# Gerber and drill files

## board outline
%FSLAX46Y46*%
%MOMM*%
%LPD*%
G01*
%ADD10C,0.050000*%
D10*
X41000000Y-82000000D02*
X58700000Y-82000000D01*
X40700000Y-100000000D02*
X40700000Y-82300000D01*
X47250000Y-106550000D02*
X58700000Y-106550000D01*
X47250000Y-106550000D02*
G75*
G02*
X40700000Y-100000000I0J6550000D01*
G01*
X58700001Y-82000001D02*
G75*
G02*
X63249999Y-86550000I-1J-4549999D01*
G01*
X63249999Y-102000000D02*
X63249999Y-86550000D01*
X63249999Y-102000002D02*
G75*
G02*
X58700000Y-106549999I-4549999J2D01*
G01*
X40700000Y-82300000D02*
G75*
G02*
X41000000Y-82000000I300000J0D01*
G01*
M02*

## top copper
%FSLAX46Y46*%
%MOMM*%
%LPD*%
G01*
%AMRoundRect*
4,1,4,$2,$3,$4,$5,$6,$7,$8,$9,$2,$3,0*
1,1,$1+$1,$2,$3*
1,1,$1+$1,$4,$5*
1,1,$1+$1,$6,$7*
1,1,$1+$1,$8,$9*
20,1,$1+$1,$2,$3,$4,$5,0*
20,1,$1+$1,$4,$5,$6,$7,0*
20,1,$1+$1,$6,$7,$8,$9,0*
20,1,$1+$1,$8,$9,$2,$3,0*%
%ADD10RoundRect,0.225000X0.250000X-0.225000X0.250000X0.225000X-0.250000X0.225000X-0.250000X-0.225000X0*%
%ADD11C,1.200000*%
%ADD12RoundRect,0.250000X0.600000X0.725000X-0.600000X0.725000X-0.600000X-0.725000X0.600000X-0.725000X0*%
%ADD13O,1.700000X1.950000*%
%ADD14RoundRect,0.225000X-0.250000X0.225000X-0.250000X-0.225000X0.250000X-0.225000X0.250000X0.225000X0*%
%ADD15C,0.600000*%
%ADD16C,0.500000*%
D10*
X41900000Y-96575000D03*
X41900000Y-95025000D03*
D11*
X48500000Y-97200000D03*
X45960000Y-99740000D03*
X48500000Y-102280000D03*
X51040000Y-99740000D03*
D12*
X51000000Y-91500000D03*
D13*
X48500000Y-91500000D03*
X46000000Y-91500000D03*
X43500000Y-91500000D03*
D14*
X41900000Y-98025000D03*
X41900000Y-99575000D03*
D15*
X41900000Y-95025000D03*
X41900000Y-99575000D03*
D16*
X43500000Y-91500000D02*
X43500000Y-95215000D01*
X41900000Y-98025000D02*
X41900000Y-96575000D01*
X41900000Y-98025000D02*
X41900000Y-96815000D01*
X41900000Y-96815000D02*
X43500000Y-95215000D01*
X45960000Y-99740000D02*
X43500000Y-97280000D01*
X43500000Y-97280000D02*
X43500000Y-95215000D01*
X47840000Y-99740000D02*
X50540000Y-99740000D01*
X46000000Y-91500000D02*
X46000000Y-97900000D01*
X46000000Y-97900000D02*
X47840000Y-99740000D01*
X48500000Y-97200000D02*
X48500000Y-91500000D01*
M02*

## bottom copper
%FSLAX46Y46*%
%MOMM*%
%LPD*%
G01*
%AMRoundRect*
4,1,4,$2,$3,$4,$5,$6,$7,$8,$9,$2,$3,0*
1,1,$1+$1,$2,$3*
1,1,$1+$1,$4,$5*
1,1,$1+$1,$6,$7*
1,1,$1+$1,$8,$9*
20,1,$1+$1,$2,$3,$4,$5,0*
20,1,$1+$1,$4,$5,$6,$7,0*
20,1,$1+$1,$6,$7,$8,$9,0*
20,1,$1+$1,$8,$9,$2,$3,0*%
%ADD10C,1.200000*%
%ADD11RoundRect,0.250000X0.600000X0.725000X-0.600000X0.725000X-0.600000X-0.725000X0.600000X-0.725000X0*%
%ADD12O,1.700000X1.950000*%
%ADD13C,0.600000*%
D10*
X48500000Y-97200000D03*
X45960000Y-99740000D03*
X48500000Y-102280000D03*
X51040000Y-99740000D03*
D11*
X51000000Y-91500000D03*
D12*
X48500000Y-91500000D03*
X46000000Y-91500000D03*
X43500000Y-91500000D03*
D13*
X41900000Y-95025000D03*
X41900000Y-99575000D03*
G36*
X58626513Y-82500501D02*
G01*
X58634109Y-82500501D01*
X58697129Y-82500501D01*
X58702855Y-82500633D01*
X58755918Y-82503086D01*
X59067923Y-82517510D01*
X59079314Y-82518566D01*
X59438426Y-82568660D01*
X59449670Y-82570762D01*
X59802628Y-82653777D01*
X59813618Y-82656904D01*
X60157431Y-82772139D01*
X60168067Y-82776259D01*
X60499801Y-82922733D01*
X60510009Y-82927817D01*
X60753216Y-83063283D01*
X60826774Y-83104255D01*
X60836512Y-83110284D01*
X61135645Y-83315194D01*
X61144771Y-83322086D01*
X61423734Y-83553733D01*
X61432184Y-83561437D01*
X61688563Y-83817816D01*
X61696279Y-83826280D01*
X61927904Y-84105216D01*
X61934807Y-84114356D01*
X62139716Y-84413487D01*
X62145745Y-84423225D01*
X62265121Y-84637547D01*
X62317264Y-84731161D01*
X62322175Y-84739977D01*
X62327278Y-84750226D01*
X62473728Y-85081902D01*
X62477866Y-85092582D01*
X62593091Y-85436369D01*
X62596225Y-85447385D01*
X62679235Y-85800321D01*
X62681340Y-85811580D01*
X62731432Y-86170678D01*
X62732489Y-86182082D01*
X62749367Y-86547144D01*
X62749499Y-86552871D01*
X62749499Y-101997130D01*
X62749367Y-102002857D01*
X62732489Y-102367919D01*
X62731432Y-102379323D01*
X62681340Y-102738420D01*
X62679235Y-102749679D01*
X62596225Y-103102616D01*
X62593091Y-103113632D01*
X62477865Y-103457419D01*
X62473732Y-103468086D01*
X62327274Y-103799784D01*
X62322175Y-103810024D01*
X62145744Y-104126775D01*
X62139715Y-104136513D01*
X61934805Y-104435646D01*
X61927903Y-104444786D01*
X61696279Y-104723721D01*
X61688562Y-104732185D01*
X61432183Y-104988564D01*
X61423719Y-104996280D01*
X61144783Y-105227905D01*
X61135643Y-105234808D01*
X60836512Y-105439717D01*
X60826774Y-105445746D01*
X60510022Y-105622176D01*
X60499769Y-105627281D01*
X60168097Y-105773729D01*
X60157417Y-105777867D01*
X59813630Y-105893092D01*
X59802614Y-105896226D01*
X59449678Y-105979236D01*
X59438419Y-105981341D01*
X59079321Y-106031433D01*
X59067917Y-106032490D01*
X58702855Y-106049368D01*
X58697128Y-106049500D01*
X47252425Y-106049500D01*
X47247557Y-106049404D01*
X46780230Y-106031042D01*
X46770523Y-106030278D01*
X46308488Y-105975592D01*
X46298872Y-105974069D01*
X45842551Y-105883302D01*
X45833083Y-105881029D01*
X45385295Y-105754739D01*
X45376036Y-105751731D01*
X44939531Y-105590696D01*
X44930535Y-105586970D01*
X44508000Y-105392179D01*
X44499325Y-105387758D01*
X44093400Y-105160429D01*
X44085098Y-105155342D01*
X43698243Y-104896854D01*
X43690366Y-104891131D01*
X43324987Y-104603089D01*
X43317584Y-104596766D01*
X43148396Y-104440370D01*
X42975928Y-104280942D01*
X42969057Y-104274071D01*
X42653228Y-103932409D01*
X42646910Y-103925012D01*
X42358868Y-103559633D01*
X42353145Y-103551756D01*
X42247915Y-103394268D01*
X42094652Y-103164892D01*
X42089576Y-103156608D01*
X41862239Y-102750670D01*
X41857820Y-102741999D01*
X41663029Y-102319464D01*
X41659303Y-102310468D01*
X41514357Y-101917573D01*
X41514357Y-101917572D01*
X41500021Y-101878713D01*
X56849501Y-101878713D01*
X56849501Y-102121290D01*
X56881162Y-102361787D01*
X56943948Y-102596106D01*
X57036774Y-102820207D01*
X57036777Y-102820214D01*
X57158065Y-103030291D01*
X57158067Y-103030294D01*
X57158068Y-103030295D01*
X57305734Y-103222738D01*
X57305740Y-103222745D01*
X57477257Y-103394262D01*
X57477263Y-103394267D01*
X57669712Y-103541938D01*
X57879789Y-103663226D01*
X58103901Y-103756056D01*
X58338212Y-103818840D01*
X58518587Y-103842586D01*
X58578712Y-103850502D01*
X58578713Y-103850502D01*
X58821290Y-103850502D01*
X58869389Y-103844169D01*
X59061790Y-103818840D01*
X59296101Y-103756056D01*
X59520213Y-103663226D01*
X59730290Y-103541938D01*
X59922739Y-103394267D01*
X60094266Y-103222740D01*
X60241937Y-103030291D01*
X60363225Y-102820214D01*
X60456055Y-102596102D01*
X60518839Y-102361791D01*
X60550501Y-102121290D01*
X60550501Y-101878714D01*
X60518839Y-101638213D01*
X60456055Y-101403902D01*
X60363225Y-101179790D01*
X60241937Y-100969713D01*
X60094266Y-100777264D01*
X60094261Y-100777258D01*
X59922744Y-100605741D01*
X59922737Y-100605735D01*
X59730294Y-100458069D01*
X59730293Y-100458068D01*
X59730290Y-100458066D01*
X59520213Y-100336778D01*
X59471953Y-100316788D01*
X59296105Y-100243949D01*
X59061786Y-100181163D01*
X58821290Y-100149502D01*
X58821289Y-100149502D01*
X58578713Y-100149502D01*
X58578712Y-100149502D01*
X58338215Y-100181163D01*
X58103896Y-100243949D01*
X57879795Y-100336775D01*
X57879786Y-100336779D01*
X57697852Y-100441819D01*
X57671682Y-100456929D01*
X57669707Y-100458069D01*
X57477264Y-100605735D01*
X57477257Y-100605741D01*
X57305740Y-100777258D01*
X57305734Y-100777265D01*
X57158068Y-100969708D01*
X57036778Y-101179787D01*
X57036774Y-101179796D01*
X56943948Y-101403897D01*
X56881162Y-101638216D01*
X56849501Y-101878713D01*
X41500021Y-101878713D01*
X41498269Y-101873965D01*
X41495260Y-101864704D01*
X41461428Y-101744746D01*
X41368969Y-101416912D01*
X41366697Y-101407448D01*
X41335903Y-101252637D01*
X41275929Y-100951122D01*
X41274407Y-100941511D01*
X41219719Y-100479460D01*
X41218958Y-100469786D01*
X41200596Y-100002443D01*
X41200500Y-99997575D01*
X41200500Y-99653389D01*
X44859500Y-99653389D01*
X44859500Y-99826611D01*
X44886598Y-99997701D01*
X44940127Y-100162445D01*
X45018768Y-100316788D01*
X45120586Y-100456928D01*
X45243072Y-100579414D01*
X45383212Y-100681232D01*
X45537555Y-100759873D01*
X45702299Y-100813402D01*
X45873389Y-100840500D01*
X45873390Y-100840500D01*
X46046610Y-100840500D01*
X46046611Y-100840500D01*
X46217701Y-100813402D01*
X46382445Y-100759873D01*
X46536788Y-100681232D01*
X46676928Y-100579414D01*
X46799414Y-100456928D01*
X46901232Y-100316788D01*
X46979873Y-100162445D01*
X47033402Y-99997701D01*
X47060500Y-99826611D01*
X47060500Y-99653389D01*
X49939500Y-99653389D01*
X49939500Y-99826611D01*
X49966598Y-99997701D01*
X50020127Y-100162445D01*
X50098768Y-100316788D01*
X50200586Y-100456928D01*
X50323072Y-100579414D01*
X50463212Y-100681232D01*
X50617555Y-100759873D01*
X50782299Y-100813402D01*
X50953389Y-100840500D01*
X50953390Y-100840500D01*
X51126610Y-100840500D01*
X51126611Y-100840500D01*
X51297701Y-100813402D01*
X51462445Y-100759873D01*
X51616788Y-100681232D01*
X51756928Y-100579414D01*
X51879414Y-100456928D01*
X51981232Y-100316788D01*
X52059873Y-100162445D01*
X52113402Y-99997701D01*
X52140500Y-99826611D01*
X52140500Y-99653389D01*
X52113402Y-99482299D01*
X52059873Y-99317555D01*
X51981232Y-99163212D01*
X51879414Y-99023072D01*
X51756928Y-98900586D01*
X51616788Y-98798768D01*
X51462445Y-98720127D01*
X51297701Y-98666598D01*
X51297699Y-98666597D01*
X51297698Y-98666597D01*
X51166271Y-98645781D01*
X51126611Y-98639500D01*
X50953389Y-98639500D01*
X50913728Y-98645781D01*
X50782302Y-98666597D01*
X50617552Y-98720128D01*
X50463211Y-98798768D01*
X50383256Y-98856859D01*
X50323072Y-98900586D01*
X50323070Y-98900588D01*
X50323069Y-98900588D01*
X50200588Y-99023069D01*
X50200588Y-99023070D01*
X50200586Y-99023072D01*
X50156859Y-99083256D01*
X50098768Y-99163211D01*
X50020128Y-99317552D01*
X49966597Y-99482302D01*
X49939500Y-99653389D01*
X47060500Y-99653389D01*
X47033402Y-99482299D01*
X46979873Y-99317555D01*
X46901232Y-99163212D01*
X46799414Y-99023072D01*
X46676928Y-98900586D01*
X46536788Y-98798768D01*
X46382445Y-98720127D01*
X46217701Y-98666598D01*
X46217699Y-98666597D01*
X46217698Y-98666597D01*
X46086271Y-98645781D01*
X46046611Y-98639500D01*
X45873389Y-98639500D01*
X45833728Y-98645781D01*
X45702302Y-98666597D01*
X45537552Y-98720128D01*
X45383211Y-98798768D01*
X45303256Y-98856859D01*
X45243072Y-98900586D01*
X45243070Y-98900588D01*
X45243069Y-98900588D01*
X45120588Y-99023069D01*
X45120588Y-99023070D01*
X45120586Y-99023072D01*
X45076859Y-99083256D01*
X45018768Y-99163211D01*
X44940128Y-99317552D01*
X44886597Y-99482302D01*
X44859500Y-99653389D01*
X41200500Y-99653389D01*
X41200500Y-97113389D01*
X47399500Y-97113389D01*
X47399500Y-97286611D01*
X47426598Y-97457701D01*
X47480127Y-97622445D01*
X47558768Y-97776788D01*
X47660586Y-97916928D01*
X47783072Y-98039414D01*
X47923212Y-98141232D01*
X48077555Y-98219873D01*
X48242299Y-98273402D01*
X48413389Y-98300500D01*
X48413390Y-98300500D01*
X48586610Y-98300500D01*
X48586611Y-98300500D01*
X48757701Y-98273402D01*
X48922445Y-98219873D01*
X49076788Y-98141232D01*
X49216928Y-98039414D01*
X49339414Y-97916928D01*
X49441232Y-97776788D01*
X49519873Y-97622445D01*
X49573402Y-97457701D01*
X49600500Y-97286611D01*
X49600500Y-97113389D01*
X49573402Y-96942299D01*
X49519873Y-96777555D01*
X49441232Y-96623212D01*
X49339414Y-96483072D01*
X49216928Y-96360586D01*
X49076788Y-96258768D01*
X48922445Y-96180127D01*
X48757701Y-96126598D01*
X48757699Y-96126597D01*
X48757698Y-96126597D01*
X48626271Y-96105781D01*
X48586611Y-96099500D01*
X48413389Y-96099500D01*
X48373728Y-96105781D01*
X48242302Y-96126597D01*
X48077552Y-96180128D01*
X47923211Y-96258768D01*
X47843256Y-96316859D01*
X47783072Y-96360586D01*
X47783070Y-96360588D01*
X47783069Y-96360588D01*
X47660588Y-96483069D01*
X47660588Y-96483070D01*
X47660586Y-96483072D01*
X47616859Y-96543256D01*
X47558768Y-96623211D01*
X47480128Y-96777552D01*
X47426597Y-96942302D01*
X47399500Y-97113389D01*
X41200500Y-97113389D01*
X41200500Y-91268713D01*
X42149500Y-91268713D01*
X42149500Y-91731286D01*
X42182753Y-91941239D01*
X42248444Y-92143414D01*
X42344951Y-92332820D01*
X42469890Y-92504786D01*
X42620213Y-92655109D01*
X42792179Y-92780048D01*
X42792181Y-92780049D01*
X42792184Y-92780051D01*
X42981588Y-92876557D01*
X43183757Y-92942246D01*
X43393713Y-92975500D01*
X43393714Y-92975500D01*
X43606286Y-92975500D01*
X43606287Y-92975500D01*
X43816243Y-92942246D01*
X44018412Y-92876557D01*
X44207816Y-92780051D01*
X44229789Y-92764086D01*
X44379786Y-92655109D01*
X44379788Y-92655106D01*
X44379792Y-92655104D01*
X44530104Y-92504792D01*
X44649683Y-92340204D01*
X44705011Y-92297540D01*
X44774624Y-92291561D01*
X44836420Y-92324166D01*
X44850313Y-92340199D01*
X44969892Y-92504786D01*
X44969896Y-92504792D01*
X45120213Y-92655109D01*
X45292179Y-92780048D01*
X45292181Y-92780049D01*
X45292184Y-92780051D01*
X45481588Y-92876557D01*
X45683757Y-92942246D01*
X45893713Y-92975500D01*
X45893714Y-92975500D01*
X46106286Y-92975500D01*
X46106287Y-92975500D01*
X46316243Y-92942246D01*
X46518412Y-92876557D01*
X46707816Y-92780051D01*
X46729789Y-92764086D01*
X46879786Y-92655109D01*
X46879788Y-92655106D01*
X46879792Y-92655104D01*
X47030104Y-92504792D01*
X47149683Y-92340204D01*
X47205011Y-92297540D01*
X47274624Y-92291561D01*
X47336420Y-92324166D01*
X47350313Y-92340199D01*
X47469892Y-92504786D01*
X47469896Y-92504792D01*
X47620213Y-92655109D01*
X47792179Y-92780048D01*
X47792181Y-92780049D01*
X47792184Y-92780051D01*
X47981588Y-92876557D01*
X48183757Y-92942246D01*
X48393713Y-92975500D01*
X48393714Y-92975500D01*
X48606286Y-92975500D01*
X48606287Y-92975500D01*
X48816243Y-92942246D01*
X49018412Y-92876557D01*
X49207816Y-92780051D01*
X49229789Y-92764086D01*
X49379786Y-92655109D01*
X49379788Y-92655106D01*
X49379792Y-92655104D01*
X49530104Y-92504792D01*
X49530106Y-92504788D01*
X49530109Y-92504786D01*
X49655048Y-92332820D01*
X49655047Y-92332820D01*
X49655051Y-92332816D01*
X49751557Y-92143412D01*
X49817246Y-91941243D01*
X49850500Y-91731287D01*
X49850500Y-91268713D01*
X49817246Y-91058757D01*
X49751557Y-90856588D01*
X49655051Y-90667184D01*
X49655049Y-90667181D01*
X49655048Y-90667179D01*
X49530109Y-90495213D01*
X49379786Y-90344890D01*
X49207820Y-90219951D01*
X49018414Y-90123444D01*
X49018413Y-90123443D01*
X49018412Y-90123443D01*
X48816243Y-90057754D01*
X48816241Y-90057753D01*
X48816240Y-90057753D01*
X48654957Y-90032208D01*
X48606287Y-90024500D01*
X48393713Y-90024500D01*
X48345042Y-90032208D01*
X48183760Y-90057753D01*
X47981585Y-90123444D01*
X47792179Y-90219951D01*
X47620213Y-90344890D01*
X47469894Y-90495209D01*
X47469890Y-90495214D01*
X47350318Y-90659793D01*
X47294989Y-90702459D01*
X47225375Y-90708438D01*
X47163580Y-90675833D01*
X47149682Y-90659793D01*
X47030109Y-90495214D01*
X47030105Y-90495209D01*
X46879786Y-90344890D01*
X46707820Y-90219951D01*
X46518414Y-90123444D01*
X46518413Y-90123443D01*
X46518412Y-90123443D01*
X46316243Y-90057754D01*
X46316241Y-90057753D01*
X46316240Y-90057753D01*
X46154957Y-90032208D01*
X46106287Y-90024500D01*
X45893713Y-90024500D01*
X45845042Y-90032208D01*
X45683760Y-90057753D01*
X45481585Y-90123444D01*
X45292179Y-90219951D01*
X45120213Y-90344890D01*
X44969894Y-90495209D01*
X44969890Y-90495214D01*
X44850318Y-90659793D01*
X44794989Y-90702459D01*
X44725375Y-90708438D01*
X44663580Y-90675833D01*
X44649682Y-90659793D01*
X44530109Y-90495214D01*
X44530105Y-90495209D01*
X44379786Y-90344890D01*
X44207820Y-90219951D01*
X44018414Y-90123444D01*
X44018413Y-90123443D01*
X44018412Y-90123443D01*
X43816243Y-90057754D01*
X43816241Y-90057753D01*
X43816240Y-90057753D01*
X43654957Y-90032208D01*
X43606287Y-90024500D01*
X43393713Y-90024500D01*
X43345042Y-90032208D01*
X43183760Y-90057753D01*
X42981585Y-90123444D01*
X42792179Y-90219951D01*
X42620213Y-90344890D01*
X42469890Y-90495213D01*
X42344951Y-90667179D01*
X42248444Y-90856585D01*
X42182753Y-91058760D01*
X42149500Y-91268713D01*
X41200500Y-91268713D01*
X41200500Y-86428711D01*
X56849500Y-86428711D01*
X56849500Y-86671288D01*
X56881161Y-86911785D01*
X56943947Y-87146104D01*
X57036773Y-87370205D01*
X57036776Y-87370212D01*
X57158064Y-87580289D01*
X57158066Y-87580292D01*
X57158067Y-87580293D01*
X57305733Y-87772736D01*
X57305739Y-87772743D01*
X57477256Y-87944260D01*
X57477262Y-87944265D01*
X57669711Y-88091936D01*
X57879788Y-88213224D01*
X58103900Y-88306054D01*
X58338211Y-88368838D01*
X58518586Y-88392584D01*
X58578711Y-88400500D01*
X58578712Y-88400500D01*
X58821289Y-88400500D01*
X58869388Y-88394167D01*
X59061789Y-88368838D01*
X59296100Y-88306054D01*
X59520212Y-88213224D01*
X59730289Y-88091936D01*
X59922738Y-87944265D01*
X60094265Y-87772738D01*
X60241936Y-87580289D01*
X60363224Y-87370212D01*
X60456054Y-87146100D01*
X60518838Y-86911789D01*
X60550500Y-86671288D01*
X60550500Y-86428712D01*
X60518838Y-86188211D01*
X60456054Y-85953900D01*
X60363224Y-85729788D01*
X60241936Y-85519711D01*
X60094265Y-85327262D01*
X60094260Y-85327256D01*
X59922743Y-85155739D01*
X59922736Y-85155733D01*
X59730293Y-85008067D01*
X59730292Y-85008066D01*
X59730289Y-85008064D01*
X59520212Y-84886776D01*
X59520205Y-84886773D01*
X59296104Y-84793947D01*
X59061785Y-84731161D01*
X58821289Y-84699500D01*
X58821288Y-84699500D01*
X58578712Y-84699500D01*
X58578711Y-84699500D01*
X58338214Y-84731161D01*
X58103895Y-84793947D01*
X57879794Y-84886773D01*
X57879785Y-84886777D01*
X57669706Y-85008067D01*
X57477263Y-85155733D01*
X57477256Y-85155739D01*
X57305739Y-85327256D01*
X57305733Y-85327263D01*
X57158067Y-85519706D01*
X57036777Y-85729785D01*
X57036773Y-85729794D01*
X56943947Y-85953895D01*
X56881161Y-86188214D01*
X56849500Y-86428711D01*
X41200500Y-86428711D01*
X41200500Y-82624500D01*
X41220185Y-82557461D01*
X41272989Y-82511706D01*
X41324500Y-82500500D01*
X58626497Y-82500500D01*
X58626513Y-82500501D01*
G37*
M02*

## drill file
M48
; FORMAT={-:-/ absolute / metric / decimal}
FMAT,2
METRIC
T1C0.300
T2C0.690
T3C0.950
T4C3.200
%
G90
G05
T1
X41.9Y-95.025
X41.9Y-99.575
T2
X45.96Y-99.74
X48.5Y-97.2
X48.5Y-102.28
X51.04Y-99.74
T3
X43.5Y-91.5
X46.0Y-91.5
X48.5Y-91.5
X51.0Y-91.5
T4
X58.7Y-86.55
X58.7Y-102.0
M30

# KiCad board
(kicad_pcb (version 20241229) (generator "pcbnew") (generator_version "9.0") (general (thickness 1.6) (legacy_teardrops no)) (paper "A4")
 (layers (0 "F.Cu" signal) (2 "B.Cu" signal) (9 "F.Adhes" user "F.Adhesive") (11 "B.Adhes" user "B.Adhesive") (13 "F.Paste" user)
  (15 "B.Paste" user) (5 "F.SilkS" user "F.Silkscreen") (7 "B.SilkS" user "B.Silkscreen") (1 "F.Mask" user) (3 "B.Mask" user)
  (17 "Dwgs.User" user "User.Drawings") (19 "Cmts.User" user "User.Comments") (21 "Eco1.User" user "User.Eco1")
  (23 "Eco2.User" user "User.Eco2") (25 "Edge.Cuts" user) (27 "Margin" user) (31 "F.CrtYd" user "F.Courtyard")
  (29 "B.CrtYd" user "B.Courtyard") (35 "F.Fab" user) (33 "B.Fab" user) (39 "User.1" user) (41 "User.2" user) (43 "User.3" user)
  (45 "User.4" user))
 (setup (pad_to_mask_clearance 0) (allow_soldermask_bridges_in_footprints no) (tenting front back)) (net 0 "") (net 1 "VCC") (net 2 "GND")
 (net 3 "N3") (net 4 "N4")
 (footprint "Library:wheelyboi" (layer "F.Cu") (at 61.05 89.3 -90)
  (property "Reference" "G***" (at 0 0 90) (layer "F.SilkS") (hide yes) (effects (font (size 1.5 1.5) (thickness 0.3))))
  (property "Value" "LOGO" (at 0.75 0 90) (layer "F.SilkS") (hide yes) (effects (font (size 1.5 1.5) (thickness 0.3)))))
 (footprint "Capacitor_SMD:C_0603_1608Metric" (layer "F.Cu") (at 41.9 95.8 90)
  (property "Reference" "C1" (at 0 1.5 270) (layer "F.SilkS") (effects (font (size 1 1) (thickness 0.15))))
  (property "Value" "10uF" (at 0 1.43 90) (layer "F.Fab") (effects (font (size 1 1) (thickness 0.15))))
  (pad "1" smd roundrect (at -0.775 0 90) (size 0.9 0.95) (layers "F.Cu" "F.Mask" "F.Paste") (roundrect_rratio 0.25) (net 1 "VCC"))
  (pad "2" smd roundrect (at 0.775 0 90) (size 0.9 0.95) (layers "F.Cu" "F.Mask" "F.Paste") (roundrect_rratio 0.25) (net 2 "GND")))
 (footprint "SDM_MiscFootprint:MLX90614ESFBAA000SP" (layer "F.Cu") (at 48.5 97.2 -90)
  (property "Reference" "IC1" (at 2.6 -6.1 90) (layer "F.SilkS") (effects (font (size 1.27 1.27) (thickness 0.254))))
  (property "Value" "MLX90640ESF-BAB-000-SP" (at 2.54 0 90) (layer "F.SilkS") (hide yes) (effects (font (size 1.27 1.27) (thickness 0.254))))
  (pad "1" thru_hole circle (at 0 0 270) (size 1.2 1.2) (drill 0.69) (layers "*.Cu" "*.Mask") (remove_unused_layers no) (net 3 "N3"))
  (pad "2" thru_hole circle (at 2.54 2.54 270) (size 1.2 1.2) (drill 0.69) (layers "*.Cu" "*.Mask") (remove_unused_layers no) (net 1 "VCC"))
  (pad "3" thru_hole circle (at 5.08 0 270) (size 1.2 1.2) (drill 0.69) (layers "*.Cu" "*.Mask") (remove_unused_layers no) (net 2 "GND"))
  (pad "4" thru_hole circle (at 2.54 -2.54 270) (size 1.2 1.2) (drill 0.69) (layers "*.Cu" "*.Mask") (remove_unused_layers no) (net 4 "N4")))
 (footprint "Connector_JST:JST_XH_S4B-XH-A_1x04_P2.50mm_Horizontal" (layer "F.Cu") (at 51 91.5 180)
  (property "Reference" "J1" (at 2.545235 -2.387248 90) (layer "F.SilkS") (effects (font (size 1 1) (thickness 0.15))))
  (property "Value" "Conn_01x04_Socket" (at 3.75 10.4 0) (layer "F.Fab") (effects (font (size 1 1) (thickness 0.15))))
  (pad "1" thru_hole roundrect (at 0 0 180) (size 1.7 1.95) (drill 0.95) (layers "*.Cu" "*.Mask") (remove_unused_layers no)
   (roundrect_rratio 0.147059) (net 2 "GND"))
  (pad "2" thru_hole oval (at 2.5 0 180) (size 1.7 1.95) (drill 0.95) (layers "*.Cu" "*.Mask") (remove_unused_layers no) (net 3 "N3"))
  (pad "3" thru_hole oval (at 5 0 180) (size 1.7 1.95) (drill 0.95) (layers "*.Cu" "*.Mask") (remove_unused_layers no) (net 4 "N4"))
  (pad "4" thru_hole oval (at 7.5 0 180) (size 1.7 1.95) (drill 0.95) (layers "*.Cu" "*.Mask") (remove_unused_layers no) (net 1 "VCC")))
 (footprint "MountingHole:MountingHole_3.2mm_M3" (layer "F.Cu") (at 58.7 86.55)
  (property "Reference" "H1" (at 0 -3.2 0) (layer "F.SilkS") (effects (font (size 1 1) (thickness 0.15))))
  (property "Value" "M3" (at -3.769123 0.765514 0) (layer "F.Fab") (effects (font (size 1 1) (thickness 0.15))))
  (pad "" np_thru_hole circle (at 0 0) (size 3.2 3.2) (drill 3.2) (layers "*.Cu" "*.Mask")))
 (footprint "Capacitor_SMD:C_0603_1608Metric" (layer "F.Cu") (at 41.9 98.8 -90)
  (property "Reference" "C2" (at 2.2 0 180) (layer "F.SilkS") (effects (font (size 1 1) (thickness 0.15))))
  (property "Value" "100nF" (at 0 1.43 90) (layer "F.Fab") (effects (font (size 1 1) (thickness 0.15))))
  (pad "1" smd roundrect (at -0.775 0 270) (size 0.9 0.95) (layers "F.Cu" "F.Mask" "F.Paste") (roundrect_rratio 0.25) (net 1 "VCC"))
  (pad "2" smd roundrect (at 0.775 0 270) (size 0.9 0.95) (layers "F.Cu" "F.Mask" "F.Paste") (roundrect_rratio 0.25) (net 2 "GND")))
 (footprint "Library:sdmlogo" (layer "F.Cu") (at 62 95.3 -90)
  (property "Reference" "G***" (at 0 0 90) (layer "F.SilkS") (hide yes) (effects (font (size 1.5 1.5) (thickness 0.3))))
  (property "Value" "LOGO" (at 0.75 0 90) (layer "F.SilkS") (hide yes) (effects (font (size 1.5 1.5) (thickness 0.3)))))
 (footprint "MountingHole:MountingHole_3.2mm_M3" (layer "F.Cu") (at 58.700001 102.000002)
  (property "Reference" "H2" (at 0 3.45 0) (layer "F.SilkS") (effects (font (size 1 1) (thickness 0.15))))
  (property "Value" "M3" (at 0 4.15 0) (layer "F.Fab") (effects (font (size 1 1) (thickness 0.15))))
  (pad "" np_thru_hole circle (at 0 0) (size 3.2 3.2) (drill 3.2) (layers "*.Cu" "*.Mask")))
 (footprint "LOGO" (layer "B.Cu") (at 47.304066 85.596581 90)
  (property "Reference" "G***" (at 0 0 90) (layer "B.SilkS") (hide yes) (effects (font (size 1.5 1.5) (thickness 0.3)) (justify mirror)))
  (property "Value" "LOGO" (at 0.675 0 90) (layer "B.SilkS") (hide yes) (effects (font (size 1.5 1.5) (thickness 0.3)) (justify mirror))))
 (gr_line (start 41 82) (end 58.7 82) (stroke (width 0.05) (type default)) (layer "Edge.Cuts"))
 (gr_line (start 40.7 100) (end 40.7 82.3) (stroke (width 0.05) (type default)) (layer "Edge.Cuts"))
 (gr_line (start 47.25 106.55) (end 58.7 106.55) (stroke (width 0.05) (type default)) (layer "Edge.Cuts"))
 (gr_arc (start 47.25 106.55) (mid 42.618451 104.631549) (end 40.7 100) (stroke (width 0.05) (type solid)) (layer "Edge.Cuts"))
 (gr_arc (start 58.700001 82.000001) (mid 61.917336 83.332665) (end 63.249999 86.55) (stroke (width 0.05) (type default))
  (layer "Edge.Cuts"))
 (gr_line (start 63.249999 102) (end 63.249999 86.55) (stroke (width 0.05) (type default)) (layer "Edge.Cuts"))
 (gr_arc (start 63.249999 102.000002) (mid 61.917335 105.217337) (end 58.7 106.55) (stroke (width 0.05) (type default)) (layer "Edge.Cuts"))
 (gr_arc (start 40.7 82.3) (mid 40.787868 82.087868) (end 41 82) (stroke (width 0.05) (type default)) (layer "Edge.Cuts"))
 (segment (start 43.5 91.5) (end 43.5 95.215) (width 0.5) (layer "F.Cu") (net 1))
 (segment (start 41.9 98.025) (end 41.9 96.575) (width 0.5) (layer "F.Cu") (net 1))
 (segment (start 41.9 98.025) (end 41.9 96.815) (width 0.5) (layer "F.Cu") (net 1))
 (segment (start 41.9 96.815) (end 43.5 95.215) (width 0.5) (layer "F.Cu") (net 1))
 (segment (start 45.96 99.74) (end 43.5 97.28) (width 0.5) (layer "F.Cu") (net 1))
 (segment (start 43.5 97.28) (end 43.5 95.215) (width 0.5) (layer "F.Cu") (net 1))
 (segment (start 47.84 99.74) (end 50.54 99.74) (width 0.5) (layer "F.Cu") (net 4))
 (segment (start 46 91.5) (end 46 97.9) (width 0.5) (layer "F.Cu") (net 4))
 (segment (start 46 97.9) (end 47.84 99.74) (width 0.5) (layer "F.Cu") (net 4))
 (via (at 41.9 95.025) (size 0.6) (drill 0.3) (layers "F.Cu" "B.Cu") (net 2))
 (via (at 41.9 99.575) (size 0.6) (drill 0.3) (layers "F.Cu" "B.Cu") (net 2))
 (segment (start 48.5 97.2) (end 48.5 91.5) (width 0.5) (layer "F.Cu") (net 3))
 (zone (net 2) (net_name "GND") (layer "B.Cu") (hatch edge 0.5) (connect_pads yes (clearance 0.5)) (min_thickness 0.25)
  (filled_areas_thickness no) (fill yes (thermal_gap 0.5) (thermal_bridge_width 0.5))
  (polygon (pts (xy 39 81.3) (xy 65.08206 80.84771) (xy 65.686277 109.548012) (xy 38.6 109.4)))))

